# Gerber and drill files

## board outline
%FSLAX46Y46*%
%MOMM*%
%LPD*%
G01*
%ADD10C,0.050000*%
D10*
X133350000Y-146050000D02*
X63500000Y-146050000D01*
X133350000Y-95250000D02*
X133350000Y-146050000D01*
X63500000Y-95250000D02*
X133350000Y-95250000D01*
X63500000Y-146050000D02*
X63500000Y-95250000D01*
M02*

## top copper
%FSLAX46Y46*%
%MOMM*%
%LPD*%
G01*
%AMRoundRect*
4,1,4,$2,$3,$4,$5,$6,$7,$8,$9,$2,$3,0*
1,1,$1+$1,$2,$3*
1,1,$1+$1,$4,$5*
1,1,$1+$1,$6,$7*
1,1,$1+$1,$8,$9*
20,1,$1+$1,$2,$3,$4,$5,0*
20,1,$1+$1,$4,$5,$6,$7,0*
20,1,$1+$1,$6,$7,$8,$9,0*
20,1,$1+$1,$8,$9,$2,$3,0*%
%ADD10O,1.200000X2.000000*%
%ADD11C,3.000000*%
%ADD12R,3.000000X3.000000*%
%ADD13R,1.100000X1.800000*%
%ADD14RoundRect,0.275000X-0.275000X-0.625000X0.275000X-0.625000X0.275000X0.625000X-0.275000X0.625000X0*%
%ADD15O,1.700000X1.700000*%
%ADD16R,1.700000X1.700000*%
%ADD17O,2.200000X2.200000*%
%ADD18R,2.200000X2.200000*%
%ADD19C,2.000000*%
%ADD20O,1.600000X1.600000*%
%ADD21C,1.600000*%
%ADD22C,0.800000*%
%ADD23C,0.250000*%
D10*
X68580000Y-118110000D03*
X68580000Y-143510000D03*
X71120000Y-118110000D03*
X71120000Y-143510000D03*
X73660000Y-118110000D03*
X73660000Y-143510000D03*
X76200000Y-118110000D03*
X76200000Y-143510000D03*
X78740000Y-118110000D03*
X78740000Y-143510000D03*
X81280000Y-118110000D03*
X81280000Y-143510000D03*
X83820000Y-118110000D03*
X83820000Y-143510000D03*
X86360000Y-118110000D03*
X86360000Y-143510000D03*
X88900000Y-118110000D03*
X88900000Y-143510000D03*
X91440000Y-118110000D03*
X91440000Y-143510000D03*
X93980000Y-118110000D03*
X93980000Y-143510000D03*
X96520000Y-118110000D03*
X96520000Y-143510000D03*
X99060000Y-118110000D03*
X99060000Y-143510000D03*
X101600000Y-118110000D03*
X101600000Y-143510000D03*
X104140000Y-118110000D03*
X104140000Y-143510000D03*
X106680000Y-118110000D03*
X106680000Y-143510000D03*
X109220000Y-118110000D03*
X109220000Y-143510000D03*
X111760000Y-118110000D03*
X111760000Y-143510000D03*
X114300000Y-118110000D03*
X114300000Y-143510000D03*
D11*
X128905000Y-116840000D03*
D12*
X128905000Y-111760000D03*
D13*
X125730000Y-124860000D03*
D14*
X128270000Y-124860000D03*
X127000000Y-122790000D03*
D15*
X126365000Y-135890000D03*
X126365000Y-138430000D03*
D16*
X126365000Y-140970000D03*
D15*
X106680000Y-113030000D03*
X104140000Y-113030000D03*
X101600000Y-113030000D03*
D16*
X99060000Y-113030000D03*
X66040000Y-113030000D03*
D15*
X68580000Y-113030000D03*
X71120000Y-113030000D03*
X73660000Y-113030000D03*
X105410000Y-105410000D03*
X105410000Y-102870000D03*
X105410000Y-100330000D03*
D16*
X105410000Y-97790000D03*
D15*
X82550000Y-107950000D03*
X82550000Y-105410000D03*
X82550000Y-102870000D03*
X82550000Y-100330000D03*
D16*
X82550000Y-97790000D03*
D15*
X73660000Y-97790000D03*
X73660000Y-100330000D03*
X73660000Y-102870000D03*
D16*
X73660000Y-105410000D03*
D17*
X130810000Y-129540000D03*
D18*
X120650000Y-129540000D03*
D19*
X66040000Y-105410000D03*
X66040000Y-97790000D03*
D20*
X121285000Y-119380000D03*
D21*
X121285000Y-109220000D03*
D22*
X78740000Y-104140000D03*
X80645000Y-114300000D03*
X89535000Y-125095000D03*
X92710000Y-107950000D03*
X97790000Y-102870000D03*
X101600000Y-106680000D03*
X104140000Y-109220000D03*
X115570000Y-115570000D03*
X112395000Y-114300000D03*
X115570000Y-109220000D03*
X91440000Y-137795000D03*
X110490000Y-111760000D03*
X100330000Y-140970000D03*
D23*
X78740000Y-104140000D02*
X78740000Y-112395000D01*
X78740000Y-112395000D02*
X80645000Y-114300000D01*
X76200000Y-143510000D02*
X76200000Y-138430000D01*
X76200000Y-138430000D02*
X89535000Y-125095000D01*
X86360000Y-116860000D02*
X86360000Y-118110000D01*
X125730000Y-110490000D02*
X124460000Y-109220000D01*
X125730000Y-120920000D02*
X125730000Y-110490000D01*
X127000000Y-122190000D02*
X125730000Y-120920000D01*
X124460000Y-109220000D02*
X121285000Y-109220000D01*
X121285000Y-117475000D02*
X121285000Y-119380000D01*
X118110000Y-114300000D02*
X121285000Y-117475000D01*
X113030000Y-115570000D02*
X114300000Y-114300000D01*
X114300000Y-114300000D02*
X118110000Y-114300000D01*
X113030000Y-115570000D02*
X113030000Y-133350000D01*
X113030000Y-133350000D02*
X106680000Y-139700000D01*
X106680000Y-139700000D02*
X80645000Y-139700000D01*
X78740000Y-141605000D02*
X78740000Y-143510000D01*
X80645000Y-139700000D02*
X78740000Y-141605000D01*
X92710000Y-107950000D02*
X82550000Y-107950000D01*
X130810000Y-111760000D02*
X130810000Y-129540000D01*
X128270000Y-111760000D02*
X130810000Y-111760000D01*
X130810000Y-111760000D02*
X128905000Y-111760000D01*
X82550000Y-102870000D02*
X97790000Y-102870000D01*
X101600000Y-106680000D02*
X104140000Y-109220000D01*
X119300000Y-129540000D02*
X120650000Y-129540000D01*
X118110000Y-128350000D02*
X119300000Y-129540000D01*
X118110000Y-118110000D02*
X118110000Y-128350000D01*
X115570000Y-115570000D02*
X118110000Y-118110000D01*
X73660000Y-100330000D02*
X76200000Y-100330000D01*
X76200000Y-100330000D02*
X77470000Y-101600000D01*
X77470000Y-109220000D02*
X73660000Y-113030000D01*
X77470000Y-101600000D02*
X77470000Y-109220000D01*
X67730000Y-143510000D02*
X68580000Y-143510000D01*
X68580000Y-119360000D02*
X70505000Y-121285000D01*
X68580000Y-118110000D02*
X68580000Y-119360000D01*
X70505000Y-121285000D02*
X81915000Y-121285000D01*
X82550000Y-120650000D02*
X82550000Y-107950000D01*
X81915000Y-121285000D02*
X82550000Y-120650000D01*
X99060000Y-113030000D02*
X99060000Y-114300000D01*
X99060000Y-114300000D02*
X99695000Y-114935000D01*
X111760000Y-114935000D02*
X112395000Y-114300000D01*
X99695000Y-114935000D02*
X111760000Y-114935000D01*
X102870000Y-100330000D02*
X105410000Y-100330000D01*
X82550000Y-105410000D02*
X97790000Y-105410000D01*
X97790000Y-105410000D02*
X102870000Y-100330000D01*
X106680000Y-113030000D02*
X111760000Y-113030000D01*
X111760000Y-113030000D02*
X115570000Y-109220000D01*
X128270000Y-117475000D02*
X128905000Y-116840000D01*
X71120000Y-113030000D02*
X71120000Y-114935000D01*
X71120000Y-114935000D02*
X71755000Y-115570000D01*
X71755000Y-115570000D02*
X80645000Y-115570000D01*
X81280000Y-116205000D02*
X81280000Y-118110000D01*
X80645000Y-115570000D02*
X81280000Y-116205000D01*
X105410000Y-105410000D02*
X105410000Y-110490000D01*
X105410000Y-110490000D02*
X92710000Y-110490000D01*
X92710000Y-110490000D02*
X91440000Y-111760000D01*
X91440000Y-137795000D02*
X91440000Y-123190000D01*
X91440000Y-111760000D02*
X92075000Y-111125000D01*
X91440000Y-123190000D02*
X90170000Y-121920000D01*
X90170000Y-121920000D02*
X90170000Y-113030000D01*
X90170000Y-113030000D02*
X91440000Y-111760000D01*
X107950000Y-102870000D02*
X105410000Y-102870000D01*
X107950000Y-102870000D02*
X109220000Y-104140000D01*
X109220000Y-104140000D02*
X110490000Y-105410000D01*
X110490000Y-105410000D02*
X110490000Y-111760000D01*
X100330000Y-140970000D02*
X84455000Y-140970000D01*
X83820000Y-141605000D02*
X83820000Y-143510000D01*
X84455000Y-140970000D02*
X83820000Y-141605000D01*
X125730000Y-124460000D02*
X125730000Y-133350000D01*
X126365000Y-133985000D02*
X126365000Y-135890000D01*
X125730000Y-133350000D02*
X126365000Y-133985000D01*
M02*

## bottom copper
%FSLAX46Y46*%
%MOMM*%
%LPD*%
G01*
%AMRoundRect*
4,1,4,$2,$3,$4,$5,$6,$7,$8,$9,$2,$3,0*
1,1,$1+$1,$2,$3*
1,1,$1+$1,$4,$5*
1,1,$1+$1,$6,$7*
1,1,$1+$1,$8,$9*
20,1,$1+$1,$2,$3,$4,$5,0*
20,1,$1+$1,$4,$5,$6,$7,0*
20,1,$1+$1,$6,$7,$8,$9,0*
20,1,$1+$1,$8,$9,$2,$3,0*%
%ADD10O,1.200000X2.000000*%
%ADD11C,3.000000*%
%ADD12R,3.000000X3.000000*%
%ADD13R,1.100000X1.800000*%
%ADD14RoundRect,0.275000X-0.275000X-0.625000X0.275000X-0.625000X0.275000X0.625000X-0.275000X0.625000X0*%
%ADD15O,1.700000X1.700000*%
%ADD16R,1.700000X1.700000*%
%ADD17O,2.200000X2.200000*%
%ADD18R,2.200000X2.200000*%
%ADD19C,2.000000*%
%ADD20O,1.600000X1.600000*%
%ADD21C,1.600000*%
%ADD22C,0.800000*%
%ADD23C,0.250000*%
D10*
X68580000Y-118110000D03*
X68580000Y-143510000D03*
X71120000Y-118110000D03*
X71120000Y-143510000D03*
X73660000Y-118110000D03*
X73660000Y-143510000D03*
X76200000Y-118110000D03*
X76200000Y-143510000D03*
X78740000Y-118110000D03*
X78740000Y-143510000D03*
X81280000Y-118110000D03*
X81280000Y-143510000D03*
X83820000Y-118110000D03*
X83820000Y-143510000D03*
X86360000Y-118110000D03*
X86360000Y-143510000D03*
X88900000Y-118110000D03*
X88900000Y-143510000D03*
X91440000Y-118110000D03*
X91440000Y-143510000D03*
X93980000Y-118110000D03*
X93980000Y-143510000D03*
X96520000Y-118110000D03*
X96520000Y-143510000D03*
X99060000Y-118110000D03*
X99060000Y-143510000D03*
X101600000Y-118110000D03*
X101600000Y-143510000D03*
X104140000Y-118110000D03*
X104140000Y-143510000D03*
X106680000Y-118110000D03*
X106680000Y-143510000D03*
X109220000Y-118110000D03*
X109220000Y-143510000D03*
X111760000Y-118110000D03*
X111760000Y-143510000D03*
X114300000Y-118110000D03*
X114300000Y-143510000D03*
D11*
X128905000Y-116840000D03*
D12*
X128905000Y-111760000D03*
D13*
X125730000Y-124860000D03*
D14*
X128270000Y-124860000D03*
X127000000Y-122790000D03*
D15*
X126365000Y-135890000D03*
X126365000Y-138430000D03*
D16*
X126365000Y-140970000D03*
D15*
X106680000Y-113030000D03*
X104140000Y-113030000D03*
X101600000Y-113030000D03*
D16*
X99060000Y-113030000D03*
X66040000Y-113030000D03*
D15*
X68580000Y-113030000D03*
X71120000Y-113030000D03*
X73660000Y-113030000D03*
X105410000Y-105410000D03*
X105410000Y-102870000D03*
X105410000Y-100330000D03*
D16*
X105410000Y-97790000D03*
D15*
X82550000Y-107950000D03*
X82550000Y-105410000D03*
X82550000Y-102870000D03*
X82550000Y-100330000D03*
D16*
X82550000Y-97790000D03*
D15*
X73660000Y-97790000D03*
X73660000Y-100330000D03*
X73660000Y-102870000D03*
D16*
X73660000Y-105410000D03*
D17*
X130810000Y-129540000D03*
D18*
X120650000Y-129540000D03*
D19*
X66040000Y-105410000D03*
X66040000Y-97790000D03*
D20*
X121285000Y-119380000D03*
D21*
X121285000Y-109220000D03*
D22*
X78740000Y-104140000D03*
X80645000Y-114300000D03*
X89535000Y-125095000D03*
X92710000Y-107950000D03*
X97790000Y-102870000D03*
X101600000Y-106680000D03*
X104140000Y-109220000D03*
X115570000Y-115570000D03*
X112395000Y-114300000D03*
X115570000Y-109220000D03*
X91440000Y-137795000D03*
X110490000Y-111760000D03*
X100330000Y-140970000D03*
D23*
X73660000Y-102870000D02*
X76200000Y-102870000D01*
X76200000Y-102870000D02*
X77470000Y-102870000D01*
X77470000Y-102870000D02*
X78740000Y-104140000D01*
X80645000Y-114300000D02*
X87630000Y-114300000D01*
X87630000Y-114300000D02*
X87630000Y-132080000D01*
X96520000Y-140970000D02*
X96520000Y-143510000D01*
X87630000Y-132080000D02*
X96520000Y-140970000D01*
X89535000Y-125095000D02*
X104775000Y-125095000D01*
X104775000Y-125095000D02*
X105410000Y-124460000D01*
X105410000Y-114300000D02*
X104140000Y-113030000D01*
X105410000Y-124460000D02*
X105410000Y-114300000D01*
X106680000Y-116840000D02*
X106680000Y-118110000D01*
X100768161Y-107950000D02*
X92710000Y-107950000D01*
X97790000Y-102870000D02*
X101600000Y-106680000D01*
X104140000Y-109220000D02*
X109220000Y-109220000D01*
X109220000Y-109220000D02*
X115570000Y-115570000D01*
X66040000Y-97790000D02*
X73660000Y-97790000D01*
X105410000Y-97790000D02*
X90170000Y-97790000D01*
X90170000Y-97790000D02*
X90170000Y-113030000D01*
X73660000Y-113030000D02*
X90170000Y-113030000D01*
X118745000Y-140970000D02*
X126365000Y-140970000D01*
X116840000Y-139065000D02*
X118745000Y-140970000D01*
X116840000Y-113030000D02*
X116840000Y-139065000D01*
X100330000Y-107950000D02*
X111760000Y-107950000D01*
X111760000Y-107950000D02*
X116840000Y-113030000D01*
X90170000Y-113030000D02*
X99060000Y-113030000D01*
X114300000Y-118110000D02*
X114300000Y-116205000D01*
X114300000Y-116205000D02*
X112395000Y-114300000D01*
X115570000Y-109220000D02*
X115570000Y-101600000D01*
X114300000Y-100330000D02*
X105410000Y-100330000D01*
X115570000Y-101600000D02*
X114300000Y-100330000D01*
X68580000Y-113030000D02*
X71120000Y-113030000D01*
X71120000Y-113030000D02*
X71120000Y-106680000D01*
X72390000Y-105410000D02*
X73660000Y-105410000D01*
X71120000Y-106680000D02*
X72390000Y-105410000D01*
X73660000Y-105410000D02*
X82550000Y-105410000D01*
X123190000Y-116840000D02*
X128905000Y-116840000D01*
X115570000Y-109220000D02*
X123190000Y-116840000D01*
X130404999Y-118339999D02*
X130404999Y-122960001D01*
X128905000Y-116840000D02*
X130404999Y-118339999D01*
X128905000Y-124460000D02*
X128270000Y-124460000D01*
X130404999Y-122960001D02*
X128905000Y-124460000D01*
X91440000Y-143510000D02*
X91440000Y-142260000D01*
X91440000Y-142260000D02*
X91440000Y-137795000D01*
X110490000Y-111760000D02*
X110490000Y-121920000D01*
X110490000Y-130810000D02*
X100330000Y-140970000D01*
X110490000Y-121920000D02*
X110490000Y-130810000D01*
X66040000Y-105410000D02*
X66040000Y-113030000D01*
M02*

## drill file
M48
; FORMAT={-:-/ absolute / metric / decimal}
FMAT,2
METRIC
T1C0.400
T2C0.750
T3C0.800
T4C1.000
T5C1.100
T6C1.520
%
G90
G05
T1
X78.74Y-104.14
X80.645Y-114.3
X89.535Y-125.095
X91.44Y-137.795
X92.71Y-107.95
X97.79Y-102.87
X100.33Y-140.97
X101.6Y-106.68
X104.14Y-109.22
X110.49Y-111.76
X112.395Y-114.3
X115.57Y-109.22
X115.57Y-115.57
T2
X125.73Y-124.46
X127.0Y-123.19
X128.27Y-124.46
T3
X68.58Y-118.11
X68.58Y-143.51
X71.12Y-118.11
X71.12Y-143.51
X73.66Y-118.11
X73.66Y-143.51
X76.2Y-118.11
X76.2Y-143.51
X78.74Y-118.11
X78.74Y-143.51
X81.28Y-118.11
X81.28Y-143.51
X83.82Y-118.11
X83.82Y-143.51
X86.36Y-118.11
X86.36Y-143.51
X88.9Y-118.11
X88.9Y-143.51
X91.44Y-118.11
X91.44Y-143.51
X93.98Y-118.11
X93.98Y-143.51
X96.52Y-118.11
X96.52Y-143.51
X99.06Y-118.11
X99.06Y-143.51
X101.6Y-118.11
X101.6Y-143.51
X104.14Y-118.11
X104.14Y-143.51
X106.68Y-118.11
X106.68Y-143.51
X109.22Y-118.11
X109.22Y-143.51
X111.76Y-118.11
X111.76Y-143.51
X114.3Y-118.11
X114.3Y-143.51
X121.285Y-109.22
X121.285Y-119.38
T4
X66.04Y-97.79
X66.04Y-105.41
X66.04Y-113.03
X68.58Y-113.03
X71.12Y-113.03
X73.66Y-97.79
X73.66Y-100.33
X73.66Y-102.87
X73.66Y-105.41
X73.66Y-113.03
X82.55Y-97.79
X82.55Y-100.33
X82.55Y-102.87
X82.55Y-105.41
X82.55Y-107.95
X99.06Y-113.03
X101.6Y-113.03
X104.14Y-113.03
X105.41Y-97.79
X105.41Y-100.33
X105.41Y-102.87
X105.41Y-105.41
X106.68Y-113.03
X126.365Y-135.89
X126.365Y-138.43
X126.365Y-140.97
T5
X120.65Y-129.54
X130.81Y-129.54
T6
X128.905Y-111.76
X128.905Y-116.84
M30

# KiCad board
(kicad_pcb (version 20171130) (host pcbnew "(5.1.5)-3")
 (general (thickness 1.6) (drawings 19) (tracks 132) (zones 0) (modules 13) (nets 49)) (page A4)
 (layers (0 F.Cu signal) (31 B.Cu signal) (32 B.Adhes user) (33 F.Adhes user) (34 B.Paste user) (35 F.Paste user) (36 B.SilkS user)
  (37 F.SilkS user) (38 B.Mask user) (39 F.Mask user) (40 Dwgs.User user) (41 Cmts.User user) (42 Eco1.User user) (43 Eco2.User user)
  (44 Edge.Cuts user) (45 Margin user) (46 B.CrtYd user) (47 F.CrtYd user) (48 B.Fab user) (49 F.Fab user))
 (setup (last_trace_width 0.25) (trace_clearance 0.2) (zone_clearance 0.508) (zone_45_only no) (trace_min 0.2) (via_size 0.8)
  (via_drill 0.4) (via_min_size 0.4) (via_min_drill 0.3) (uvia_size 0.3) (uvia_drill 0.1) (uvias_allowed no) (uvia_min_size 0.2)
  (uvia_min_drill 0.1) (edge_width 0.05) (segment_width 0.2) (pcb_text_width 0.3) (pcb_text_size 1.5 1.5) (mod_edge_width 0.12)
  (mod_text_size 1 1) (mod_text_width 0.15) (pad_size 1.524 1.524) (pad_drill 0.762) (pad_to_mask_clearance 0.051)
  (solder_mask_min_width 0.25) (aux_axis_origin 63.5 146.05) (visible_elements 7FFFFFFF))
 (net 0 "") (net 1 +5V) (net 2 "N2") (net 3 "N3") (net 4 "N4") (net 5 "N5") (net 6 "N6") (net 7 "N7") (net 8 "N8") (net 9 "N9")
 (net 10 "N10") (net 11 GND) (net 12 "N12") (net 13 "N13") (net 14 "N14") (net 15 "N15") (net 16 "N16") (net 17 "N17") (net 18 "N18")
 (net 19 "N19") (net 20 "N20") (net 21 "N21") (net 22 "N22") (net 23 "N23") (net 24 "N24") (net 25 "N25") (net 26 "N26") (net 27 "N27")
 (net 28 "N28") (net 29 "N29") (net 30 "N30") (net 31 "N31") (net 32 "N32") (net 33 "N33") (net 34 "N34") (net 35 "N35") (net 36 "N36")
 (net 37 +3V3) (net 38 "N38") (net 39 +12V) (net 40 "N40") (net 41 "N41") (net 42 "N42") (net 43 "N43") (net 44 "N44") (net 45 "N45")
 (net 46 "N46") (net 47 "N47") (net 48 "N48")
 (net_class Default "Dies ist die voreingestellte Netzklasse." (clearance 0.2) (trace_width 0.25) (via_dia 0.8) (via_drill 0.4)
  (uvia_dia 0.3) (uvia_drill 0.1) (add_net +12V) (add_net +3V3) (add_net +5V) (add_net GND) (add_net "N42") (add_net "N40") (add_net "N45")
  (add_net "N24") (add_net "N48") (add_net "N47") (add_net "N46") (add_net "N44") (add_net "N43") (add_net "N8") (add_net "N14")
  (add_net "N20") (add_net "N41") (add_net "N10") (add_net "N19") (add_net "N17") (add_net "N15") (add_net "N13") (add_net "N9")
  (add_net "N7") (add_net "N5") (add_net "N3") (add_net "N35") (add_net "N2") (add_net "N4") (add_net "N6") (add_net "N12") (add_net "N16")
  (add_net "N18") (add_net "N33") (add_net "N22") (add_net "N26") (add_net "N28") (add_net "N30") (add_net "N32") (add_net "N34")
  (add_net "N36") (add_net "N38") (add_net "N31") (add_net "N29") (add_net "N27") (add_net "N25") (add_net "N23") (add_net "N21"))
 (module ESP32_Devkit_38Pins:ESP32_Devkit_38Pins (layer F.Cu) (at 91.44 130.81 180)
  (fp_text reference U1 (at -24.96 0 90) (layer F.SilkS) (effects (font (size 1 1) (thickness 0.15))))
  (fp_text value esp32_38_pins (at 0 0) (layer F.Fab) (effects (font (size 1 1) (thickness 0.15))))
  (pad 19 thru_hole oval (at 22.86 12.7 180) (size 1.2 2) (drill 0.8) (layers *.Cu *.Mask) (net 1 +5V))
  (pad 20 thru_hole oval (at 22.86 -12.7 180) (size 1.2 2) (drill 0.8) (layers *.Cu *.Mask) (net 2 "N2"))
  (pad 18 thru_hole oval (at 20.32 12.7 180) (size 1.2 2) (drill 0.8) (layers *.Cu *.Mask) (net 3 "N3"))
  (pad 21 thru_hole oval (at 20.32 -12.7 180) (size 1.2 2) (drill 0.8) (layers *.Cu *.Mask) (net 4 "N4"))
  (pad 17 thru_hole oval (at 17.78 12.7 180) (size 1.2 2) (drill 0.8) (layers *.Cu *.Mask) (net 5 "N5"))
  (pad 22 thru_hole oval (at 17.78 -12.7 180) (size 1.2 2) (drill 0.8) (layers *.Cu *.Mask) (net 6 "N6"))
  (pad 16 thru_hole oval (at 15.24 12.7 180) (size 1.2 2) (drill 0.8) (layers *.Cu *.Mask) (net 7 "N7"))
  (pad 23 thru_hole oval (at 15.24 -12.7 180) (size 1.2 2) (drill 0.8) (layers *.Cu *.Mask) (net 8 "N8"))
  (pad 15 thru_hole oval (at 12.7 12.7 180) (size 1.2 2) (drill 0.8) (layers *.Cu *.Mask) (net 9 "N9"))
  (pad 24 thru_hole oval (at 12.7 -12.7 180) (size 1.2 2) (drill 0.8) (layers *.Cu *.Mask) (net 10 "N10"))
  (pad 14 thru_hole oval (at 10.16 12.7 180) (size 1.2 2) (drill 0.8) (layers *.Cu *.Mask) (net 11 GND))
  (pad 25 thru_hole oval (at 10.16 -12.7 180) (size 1.2 2) (drill 0.8) (layers *.Cu *.Mask) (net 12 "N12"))
  (pad 13 thru_hole oval (at 7.62 12.7 180) (size 1.2 2) (drill 0.8) (layers *.Cu *.Mask) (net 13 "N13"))
  (pad 26 thru_hole oval (at 7.62 -12.7 180) (size 1.2 2) (drill 0.8) (layers *.Cu *.Mask) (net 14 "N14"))
  (pad 12 thru_hole oval (at 5.08 12.7 180) (size 1.2 2) (drill 0.8) (layers *.Cu *.Mask) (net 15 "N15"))
  (pad 27 thru_hole oval (at 5.08 -12.7 180) (size 1.2 2) (drill 0.8) (layers *.Cu *.Mask) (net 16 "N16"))
  (pad 11 thru_hole oval (at 2.54 12.7 180) (size 1.2 2) (drill 0.8) (layers *.Cu *.Mask) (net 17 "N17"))
  (pad 28 thru_hole oval (at 2.54 -12.7 180) (size 1.2 2) (drill 0.8) (layers *.Cu *.Mask) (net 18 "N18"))
  (pad 10 thru_hole oval (at 0 12.7 180) (size 1.2 2) (drill 0.8) (layers *.Cu *.Mask) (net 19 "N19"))
  (pad 29 thru_hole oval (at 0 -12.7 180) (size 1.2 2) (drill 0.8) (layers *.Cu *.Mask) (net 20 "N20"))
  (pad 9 thru_hole oval (at -2.54 12.7 180) (size 1.2 2) (drill 0.8) (layers *.Cu *.Mask) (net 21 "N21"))
  (pad 30 thru_hole oval (at -2.54 -12.7 180) (size 1.2 2) (drill 0.8) (layers *.Cu *.Mask) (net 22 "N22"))
  (pad 8 thru_hole oval (at -5.08 12.7 180) (size 1.2 2) (drill 0.8) (layers *.Cu *.Mask) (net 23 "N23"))
  (pad 31 thru_hole oval (at -5.08 -12.7 180) (size 1.2 2) (drill 0.8) (layers *.Cu *.Mask) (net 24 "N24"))
  (pad 7 thru_hole oval (at -7.62 12.7 180) (size 1.2 2) (drill 0.8) (layers *.Cu *.Mask) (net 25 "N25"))
  (pad 32 thru_hole oval (at -7.62 -12.7 180) (size 1.2 2) (drill 0.8) (layers *.Cu *.Mask) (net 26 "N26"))
  (pad 6 thru_hole oval (at -10.16 12.7 180) (size 1.2 2) (drill 0.8) (layers *.Cu *.Mask) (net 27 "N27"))
  (pad 33 thru_hole oval (at -10.16 -12.7 180) (size 1.2 2) (drill 0.8) (layers *.Cu *.Mask) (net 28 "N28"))
  (pad 5 thru_hole oval (at -12.7 12.7 180) (size 1.2 2) (drill 0.8) (layers *.Cu *.Mask) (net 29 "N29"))
  (pad 34 thru_hole oval (at -12.7 -12.7 180) (size 1.2 2) (drill 0.8) (layers *.Cu *.Mask) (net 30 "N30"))
  (pad 4 thru_hole oval (at -15.24 12.7 180) (size 1.2 2) (drill 0.8) (layers *.Cu *.Mask) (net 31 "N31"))
  (pad 35 thru_hole oval (at -15.24 -12.7 180) (size 1.2 2) (drill 0.8) (layers *.Cu *.Mask) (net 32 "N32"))
  (pad 3 thru_hole oval (at -17.78 12.7 180) (size 1.2 2) (drill 0.8) (layers *.Cu *.Mask) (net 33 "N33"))
  (pad 36 thru_hole oval (at -17.78 -12.7 180) (size 1.2 2) (drill 0.8) (layers *.Cu *.Mask) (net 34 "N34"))
  (pad 2 thru_hole oval (at -20.32 12.7 180) (size 1.2 2) (drill 0.8) (layers *.Cu *.Mask) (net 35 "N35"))
  (pad 37 thru_hole oval (at -20.32 -12.7 180) (size 1.2 2) (drill 0.8) (layers *.Cu *.Mask) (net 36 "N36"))
  (pad 1 thru_hole oval (at -22.86 12.7 180) (size 1.2 2) (drill 0.8) (layers *.Cu *.Mask) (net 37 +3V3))
  (pad 38 thru_hole oval (at -22.86 -12.7 180) (size 1.2 2) (drill 0.8) (layers *.Cu *.Mask) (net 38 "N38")))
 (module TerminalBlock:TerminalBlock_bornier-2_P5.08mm (layer F.Cu) (at 128.905 111.76 270)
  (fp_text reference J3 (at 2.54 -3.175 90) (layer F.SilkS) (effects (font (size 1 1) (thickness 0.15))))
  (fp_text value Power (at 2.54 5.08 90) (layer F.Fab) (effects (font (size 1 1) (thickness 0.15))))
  (pad 2 thru_hole circle (at 5.08 0 270) (size 3 3) (drill 1.52) (layers *.Cu *.Mask) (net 11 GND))
  (pad 1 thru_hole rect (at 0 0 270) (size 3 3) (drill 1.52) (layers *.Cu *.Mask) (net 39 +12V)))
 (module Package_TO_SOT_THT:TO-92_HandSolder (layer F.Cu) (at 125.73 124.46)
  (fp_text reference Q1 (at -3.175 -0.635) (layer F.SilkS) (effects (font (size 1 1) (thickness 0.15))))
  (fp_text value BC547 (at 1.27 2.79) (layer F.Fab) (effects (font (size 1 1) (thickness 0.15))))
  (pad 1 thru_hole rect (at 0 0) (size 1.1 1.8) (drill 0.75 (offset 0 0.4)) (layers *.Cu *.Mask) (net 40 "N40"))
  (pad 3 thru_hole roundrect (at 2.54 0) (size 1.1 1.8) (drill 0.75 (offset 0 0.4)) (layers *.Cu *.Mask) (roundrect_rratio 0.25)
   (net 11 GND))
  (pad 2 thru_hole roundrect (at 1.27 -1.27) (size 1.1 1.8) (drill 0.75 (offset 0 -0.4)) (layers *.Cu *.Mask) (roundrect_rratio 0.25)
   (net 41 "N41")))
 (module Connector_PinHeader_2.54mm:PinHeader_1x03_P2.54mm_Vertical (layer F.Cu) (at 126.365 140.97 180)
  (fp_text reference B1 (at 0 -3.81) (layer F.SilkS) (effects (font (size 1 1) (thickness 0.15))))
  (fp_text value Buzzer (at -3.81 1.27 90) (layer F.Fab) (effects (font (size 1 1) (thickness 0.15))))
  (pad 3 thru_hole oval (at 0 5.08 180) (size 1.7 1.7) (drill 1) (layers *.Cu *.Mask) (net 40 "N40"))
  (pad 2 thru_hole oval (at 0 2.54 180) (size 1.7 1.7) (drill 1) (layers *.Cu *.Mask) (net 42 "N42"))
  (pad 1 thru_hole rect (at 0 0 180) (size 1.7 1.7) (drill 1) (layers *.Cu *.Mask) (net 1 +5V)))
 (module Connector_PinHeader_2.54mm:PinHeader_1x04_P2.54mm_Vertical (layer F.Cu) (at 99.06 113.03 90)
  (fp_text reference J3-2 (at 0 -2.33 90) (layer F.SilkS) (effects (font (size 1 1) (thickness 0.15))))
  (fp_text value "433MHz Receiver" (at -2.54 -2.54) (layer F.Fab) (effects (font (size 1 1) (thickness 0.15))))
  (pad 4 thru_hole oval (at 0 7.62 90) (size 1.7 1.7) (drill 1) (layers *.Cu *.Mask) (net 11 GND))
  (pad 3 thru_hole oval (at 0 5.08 90) (size 1.7 1.7) (drill 1) (layers *.Cu *.Mask) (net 8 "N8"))
  (pad 2 thru_hole oval (at 0 2.54 90) (size 1.7 1.7) (drill 1) (layers *.Cu *.Mask) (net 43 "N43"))
  (pad 1 thru_hole rect (at 0 0 90) (size 1.7 1.7) (drill 1) (layers *.Cu *.Mask) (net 37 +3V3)))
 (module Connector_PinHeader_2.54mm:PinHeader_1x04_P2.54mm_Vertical (layer F.Cu) (at 66.04 113.03 90)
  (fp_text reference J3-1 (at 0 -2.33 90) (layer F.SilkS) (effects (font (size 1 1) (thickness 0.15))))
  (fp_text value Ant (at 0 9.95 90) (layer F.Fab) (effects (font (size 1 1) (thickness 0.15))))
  (pad 1 thru_hole rect (at 0 0 90) (size 1.7 1.7) (drill 1) (layers *.Cu *.Mask) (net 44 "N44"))
  (pad 2 thru_hole oval (at 0 2.54 90) (size 1.7 1.7) (drill 1) (layers *.Cu *.Mask) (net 11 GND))
  (pad 3 thru_hole oval (at 0 5.08 90) (size 1.7 1.7) (drill 1) (layers *.Cu *.Mask) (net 11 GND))
  (pad 4 thru_hole oval (at 0 7.62 90) (size 1.7 1.7) (drill 1) (layers *.Cu *.Mask) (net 37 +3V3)))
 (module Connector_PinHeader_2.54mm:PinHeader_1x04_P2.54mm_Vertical (layer F.Cu) (at 105.41 97.79)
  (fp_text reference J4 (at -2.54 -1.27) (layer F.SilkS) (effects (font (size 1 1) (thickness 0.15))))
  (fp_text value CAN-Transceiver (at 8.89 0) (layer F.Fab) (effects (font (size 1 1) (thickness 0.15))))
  (pad 4 thru_hole oval (at 0 7.62) (size 1.7 1.7) (drill 1) (layers *.Cu *.Mask) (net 20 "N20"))
  (pad 3 thru_hole oval (at 0 5.08) (size 1.7 1.7) (drill 1) (layers *.Cu *.Mask) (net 14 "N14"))
  (pad 2 thru_hole oval (at 0 2.54) (size 1.7 1.7) (drill 1) (layers *.Cu *.Mask) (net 11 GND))
  (pad 1 thru_hole rect (at 0 0) (size 1.7 1.7) (drill 1) (layers *.Cu *.Mask) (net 37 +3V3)))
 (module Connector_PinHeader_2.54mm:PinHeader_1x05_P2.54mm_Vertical (layer F.Cu) (at 82.55 97.79)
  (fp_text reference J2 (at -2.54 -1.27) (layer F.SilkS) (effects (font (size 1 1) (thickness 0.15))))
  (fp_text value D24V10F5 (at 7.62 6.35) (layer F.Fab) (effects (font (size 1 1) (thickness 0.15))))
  (pad 5 thru_hole oval (at 0 10.16) (size 1.7 1.7) (drill 1) (layers *.Cu *.Mask) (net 1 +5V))
  (pad 4 thru_hole oval (at 0 7.62) (size 1.7 1.7) (drill 1) (layers *.Cu *.Mask) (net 11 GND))
  (pad 3 thru_hole oval (at 0 5.08) (size 1.7 1.7) (drill 1) (layers *.Cu *.Mask) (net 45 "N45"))
  (pad 2 thru_hole oval (at 0 2.54) (size 1.7 1.7) (drill 1) (layers *.Cu *.Mask) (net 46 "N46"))
  (pad 1 thru_hole rect (at 0 0) (size 1.7 1.7) (drill 1) (layers *.Cu *.Mask) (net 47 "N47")))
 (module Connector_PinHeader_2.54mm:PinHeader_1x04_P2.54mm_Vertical (layer F.Cu) (at 73.66 105.41 180)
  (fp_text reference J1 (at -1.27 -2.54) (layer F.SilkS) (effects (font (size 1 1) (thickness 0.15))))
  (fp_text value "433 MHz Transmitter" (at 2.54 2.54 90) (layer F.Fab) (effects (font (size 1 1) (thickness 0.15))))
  (pad 4 thru_hole oval (at 0 7.62 180) (size 1.7 1.7) (drill 1) (layers *.Cu *.Mask) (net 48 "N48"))
  (pad 3 thru_hole oval (at 0 5.08 180) (size 1.7 1.7) (drill 1) (layers *.Cu *.Mask) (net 37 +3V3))
  (pad 2 thru_hole oval (at 0 2.54 180) (size 1.7 1.7) (drill 1) (layers *.Cu *.Mask) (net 24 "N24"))
  (pad 1 thru_hole rect (at 0 0 180) (size 1.7 1.7) (drill 1) (layers *.Cu *.Mask) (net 11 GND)))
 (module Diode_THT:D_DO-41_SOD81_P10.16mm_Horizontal (layer F.Cu) (at 120.65 129.54)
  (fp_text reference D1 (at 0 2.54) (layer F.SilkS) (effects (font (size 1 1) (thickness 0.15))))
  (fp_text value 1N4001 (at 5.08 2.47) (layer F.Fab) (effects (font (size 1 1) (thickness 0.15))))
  (pad 2 thru_hole oval (at 10.16 0) (size 2.2 2.2) (drill 1.1) (layers *.Cu *.Mask) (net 39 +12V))
  (pad 1 thru_hole rect (at 0 0) (size 2.2 2.2) (drill 1.1) (layers *.Cu *.Mask) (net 45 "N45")))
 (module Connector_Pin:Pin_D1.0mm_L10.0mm (layer F.Cu) (at 66.04 105.41)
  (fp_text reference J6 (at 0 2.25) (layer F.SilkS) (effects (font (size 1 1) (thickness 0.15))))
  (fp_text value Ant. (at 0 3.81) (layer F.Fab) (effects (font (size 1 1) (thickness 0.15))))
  (pad 1 thru_hole circle (at 0 0) (size 2 2) (drill 1) (layers *.Cu *.Mask) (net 44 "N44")))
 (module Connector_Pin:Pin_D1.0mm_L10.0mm (layer F.Cu) (at 66.04 97.79)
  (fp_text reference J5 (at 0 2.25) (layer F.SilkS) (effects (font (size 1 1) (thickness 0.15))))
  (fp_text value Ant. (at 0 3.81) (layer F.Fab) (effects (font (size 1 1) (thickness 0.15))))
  (pad 1 thru_hole circle (at 0 0) (size 2 2) (drill 1) (layers *.Cu *.Mask) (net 48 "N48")))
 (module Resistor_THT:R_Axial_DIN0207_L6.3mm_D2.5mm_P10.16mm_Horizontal (layer F.Cu) (at 121.285 109.22 270)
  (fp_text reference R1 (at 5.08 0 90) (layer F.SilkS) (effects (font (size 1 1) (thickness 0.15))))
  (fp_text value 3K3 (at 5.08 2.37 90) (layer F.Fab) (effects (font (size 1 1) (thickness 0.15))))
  (pad 2 thru_hole oval (at 10.16 0 270) (size 1.6 1.6) (drill 0.8) (layers *.Cu *.Mask) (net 10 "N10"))
  (pad 1 thru_hole circle (at 0 0 270) (size 1.6 1.6) (drill 0.8) (layers *.Cu *.Mask) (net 41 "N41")))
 (gr_line (start 133.35 146.05) (end 63.5 146.05) (layer Edge.Cuts) (width 0.05))
 (gr_line (start 133.35 95.25) (end 133.35 146.05) (layer Edge.Cuts) (width 0.05))
 (gr_line (start 63.5 95.25) (end 133.35 95.25) (layer Edge.Cuts) (width 0.05))
 (gr_line (start 63.5 146.05) (end 63.5 95.25) (layer Edge.Cuts) (width 0.05))
 (segment (start 73.66 102.87) (end 76.2 102.87) (width 0.25) (layer B.Cu) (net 24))
 (segment (start 76.2 102.87) (end 77.47 102.87) (width 0.25) (layer B.Cu) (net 24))
 (via (at 78.74 104.14) (size 0.8) (drill 0.4) (layers F.Cu B.Cu) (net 24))
 (segment (start 77.47 102.87) (end 78.74 104.14) (width 0.25) (layer B.Cu) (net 24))
 (segment (start 78.74 104.14) (end 78.74 112.395) (width 0.25) (layer F.Cu) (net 24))
 (via (at 80.645 114.3) (size 0.8) (drill 0.4) (layers F.Cu B.Cu) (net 24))
 (segment (start 78.74 112.395) (end 80.645 114.3) (width 0.25) (layer F.Cu) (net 24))
 (segment (start 80.645 114.3) (end 87.63 114.3) (width 0.25) (layer B.Cu) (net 24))
 (segment (start 87.63 114.3) (end 87.63 132.08) (width 0.25) (layer B.Cu) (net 24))
 (segment (start 96.52 140.97) (end 96.52 143.51) (width 0.25) (layer B.Cu) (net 24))
 (segment (start 87.63 132.08) (end 96.52 140.97) (width 0.25) (layer B.Cu) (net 24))
 (segment (start 76.2 143.51) (end 76.2 138.43) (width 0.25) (layer F.Cu) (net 8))
 (via (at 89.535 125.095) (size 0.8) (drill 0.4) (layers F.Cu B.Cu) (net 8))
 (segment (start 76.2 138.43) (end 89.535 125.095) (width 0.25) (layer F.Cu) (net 8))
 (segment (start 89.535 125.095) (end 104.775 125.095) (width 0.25) (layer B.Cu) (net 8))
 (segment (start 104.775 125.095) (end 105.41 124.46) (width 0.25) (layer B.Cu) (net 8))
 (segment (start 105.41 114.3) (end 104.14 113.03) (width 0.25) (layer B.Cu) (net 8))
 (segment (start 105.41 124.46) (end 105.41 114.3) (width 0.25) (layer B.Cu) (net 8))
 (segment (start 86.36 116.86) (end 86.36 118.11) (width 0.25) (layer F.Cu) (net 15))
 (segment (start 106.68 116.84) (end 106.68 118.11) (width 0.25) (layer B.Cu) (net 31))
 (segment (start 125.73 110.49) (end 124.46 109.22) (width 0.25) (layer F.Cu) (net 41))
 (segment (start 125.73 120.92) (end 125.73 110.49) (width 0.25) (layer F.Cu) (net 41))
 (segment (start 127 122.19) (end 125.73 120.92) (width 0.25) (layer F.Cu) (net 41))
 (segment (start 124.46 109.22) (end 121.285 109.22) (width 0.25) (layer F.Cu) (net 41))
 (segment (start 121.285 117.475) (end 121.285 119.38) (width 0.25) (layer F.Cu) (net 10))
 (segment (start 118.11 114.3) (end 121.285 117.475) (width 0.25) (layer F.Cu) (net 10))
 (segment (start 113.03 115.57) (end 114.3 114.3) (width 0.25) (layer F.Cu) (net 10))
 (segment (start 114.3 114.3) (end 118.11 114.3) (width 0.25) (layer F.Cu) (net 10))
 (segment (start 113.03 115.57) (end 113.03 133.35) (width 0.25) (layer F.Cu) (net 10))
 (segment (start 113.03 133.35) (end 106.68 139.7) (width 0.25) (layer F.Cu) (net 10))
 (segment (start 106.68 139.7) (end 80.645 139.7) (width 0.25) (layer F.Cu) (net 10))
 (segment (start 78.74 141.605) (end 78.74 143.51) (width 0.25) (layer F.Cu) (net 10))
 (segment (start 80.645 139.7) (end 78.74 141.605) (width 0.25) (layer F.Cu) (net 10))
 (segment (start 100.768161 107.95) (end 92.71 107.95) (width 0.25) (layer B.Cu) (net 1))
 (via (at 92.71 107.95) (size 0.8) (drill 0.4) (layers F.Cu B.Cu) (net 1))
 (segment (start 92.71 107.95) (end 82.55 107.95) (width 0.25) (layer F.Cu) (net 1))
 (segment (start 130.81 111.76) (end 130.81 129.54) (width 0.25) (layer F.Cu) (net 39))
 (segment (start 128.27 111.76) (end 130.81 111.76) (width 0.25) (layer F.Cu) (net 39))
 (segment (start 130.81 111.76) (end 128.905 111.76) (width 0.25) (layer F.Cu) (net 39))
 (segment (start 82.55 102.87) (end 97.79 102.87) (width 0.25) (layer F.Cu) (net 45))
 (via (at 97.79 102.87) (size 0.8) (drill 0.4) (layers F.Cu B.Cu) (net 45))
 (segment (start 97.79 102.87) (end 101.6 106.68) (width 0.25) (layer B.Cu) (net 45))
 (via (at 101.6 106.68) (size 0.8) (drill 0.4) (layers F.Cu B.Cu) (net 45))
 (segment (start 101.6 106.68) (end 104.14 109.22) (width 0.25) (layer F.Cu) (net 45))
 (via (at 104.14 109.22) (size 0.8) (drill 0.4) (layers F.Cu B.Cu) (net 45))
 (segment (start 104.14 109.22) (end 109.22 109.22) (width 0.25) (layer B.Cu) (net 45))
 (segment (start 109.22 109.22) (end 115.57 115.57) (width 0.25) (layer B.Cu) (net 45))
 (via (at 115.57 115.57) (size 0.8) (drill 0.4) (layers F.Cu B.Cu) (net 45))
 (segment (start 119.3 129.54) (end 120.65 129.54) (width 0.25) (layer F.Cu) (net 45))
 (segment (start 118.11 128.35) (end 119.3 129.54) (width 0.25) (layer F.Cu) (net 45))
 (segment (start 118.11 118.11) (end 118.11 128.35) (width 0.25) (layer F.Cu) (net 45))
 (segment (start 115.57 115.57) (end 118.11 118.11) (width 0.25) (layer F.Cu) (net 45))
 (segment (start 66.04 97.79) (end 73.66 97.79) (width 0.25) (layer B.Cu) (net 48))
 (segment (start 105.41 97.79) (end 90.17 97.79) (width 0.25) (layer B.Cu) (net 37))
 (segment (start 90.17 97.79) (end 90.17 113.03) (width 0.25) (layer B.Cu) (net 37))
 (segment (start 73.66 113.03) (end 90.17 113.03) (width 0.25) (layer B.Cu) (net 37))
 (segment (start 73.66 100.33) (end 76.2 100.33) (width 0.25) (layer F.Cu) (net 37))
 (segment (start 76.2 100.33) (end 77.47 101.6) (width 0.25) (layer F.Cu) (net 37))
 (segment (start 77.47 109.22) (end 73.66 113.03) (width 0.25) (layer F.Cu) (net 37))
 (segment (start 77.47 101.6) (end 77.47 109.22) (width 0.25) (layer F.Cu) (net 37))
 (segment (start 67.73 143.51) (end 68.58 143.51) (width 0.25) (layer F.Cu) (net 2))
 (segment (start 68.58 119.36) (end 70.505 121.285) (width 0.25) (layer F.Cu) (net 1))
 (segment (start 68.58 118.11) (end 68.58 119.36) (width 0.25) (layer F.Cu) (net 1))
 (segment (start 70.505 121.285) (end 81.915 121.285) (width 0.25) (layer F.Cu) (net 1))
 (segment (start 82.55 120.65) (end 82.55 107.95) (width 0.25) (layer F.Cu) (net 1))
 (segment (start 81.915 121.285) (end 82.55 120.65) (width 0.25) (layer F.Cu) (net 1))
 (segment (start 118.745 140.97) (end 126.365 140.97) (width 0.25) (layer B.Cu) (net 1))
 (segment (start 116.84 139.065) (end 118.745 140.97) (width 0.25) (layer B.Cu) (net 1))
 (segment (start 116.84 113.03) (end 116.84 139.065) (width 0.25) (layer B.Cu) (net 1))
 (segment (start 100.33 107.95) (end 111.76 107.95) (width 0.25) (layer B.Cu) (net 1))
 (segment (start 111.76 107.95) (end 116.84 113.03) (width 0.25) (layer B.Cu) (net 1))
 (segment (start 90.17 113.03) (end 99.06 113.03) (width 0.25) (layer B.Cu) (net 37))
 (segment (start 114.3 118.11) (end 114.3 116.205) (width 0.25) (layer B.Cu) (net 37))
 (segment (start 114.3 116.205) (end 112.395 114.3) (width 0.25) (layer B.Cu) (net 37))
 (via (at 112.395 114.3) (size 0.8) (drill 0.4) (layers F.Cu B.Cu) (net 37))
 (segment (start 99.06 113.03) (end 99.06 114.3) (width 0.25) (layer F.Cu) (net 37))
 (segment (start 99.06 114.3) (end 99.695 114.935) (width 0.25) (layer F.Cu) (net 37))
 (segment (start 111.76 114.935) (end 112.395 114.3) (width 0.25) (layer F.Cu) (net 37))
 (segment (start 99.695 114.935) (end 111.76 114.935) (width 0.25) (layer F.Cu) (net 37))
 (segment (start 115.57 109.22) (end 115.57 101.6) (width 0.25) (layer B.Cu) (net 11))
 (segment (start 114.3 100.33) (end 105.41 100.33) (width 0.25) (layer B.Cu) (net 11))
 (segment (start 115.57 101.6) (end 114.3 100.33) (width 0.25) (layer B.Cu) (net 11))
 (segment (start 68.58 113.03) (end 71.12 113.03) (width 0.25) (layer B.Cu) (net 11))
 (segment (start 71.12 113.03) (end 71.12 106.68) (width 0.25) (layer B.Cu) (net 11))
 (segment (start 72.39 105.41) (end 73.66 105.41) (width 0.25) (layer B.Cu) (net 11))
 (segment (start 71.12 106.68) (end 72.39 105.41) (width 0.25) (layer B.Cu) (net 11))
 (segment (start 73.66 105.41) (end 82.55 105.41) (width 0.25) (layer B.Cu) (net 11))
 (segment (start 102.87 100.33) (end 105.41 100.33) (width 0.25) (layer F.Cu) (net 11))
 (segment (start 82.55 105.41) (end 97.79 105.41) (width 0.25) (layer F.Cu) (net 11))
 (segment (start 97.79 105.41) (end 102.87 100.33) (width 0.25) (layer F.Cu) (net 11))
 (segment (start 106.68 113.03) (end 111.76 113.03) (width 0.25) (layer F.Cu) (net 11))
 (segment (start 111.76 113.03) (end 115.57 109.22) (width 0.25) (layer F.Cu) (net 11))
 (via (at 115.57 109.22) (size 0.8) (drill 0.4) (layers F.Cu B.Cu) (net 11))
 (segment (start 123.19 116.84) (end 128.905 116.84) (width 0.25) (layer B.Cu) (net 11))
 (segment (start 115.57 109.22) (end 123.19 116.84) (width 0.25) (layer B.Cu) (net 11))
 (segment (start 128.27 117.475) (end 128.905 116.84) (width 0.25) (layer F.Cu) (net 11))
 (segment (start 130.404999 118.339999) (end 130.404999 122.960001) (width 0.25) (layer B.Cu) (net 11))
 (segment (start 128.905 116.84) (end 130.404999 118.339999) (width 0.25) (layer B.Cu) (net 11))
 (segment (start 128.905 124.46) (end 128.27 124.46) (width 0.25) (layer B.Cu) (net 11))
 (segment (start 130.404999 122.960001) (end 128.905 124.46) (width 0.25) (layer B.Cu) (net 11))
 (segment (start 71.12 113.03) (end 71.12 114.935) (width 0.25) (layer F.Cu) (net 11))
 (segment (start 71.12 114.935) (end 71.755 115.57) (width 0.25) (layer F.Cu) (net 11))
 (segment (start 71.755 115.57) (end 80.645 115.57) (width 0.25) (layer F.Cu) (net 11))
 (segment (start 81.28 116.205) (end 81.28 118.11) (width 0.25) (layer F.Cu) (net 11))
 (segment (start 80.645 115.57) (end 81.28 116.205) (width 0.25) (layer F.Cu) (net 11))
 (segment (start 105.41 105.41) (end 105.41 110.49) (width 0.25) (layer F.Cu) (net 20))
 (segment (start 105.41 110.49) (end 92.71 110.49) (width 0.25) (layer F.Cu) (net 20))
 (segment (start 92.71 110.49) (end 91.44 111.76) (width 0.25) (layer F.Cu) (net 20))
 (segment (start 91.44 143.51) (end 91.44 142.26) (width 0.25) (layer B.Cu) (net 20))
 (via (at 91.44 137.795) (size 0.8) (drill 0.4) (layers F.Cu B.Cu) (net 20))
 (segment (start 91.44 142.26) (end 91.44 137.795) (width 0.25) (layer B.Cu) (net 20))
 (segment (start 91.44 137.795) (end 91.44 123.19) (width 0.25) (layer F.Cu) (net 20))
 (segment (start 91.44 111.76) (end 92.075 111.125) (width 0.25) (layer F.Cu) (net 20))
 (segment (start 91.44 123.19) (end 90.17 121.92) (width 0.25) (layer F.Cu) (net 20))
 (segment (start 90.17 121.92) (end 90.17 113.03) (width 0.25) (layer F.Cu) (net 20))
 (segment (start 90.17 113.03) (end 91.44 111.76) (width 0.25) (layer F.Cu) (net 20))
 (segment (start 107.95 102.87) (end 105.41 102.87) (width 0.25) (layer F.Cu) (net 14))
 (segment (start 107.95 102.87) (end 109.22 104.14) (width 0.25) (layer F.Cu) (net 14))
 (segment (start 109.22 104.14) (end 110.49 105.41) (width 0.25) (layer F.Cu) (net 14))
 (via (at 110.49 111.76) (size 0.8) (drill 0.4) (layers F.Cu B.Cu) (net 14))
 (segment (start 110.49 105.41) (end 110.49 111.76) (width 0.25) (layer F.Cu) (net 14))
 (segment (start 110.49 111.76) (end 110.49 121.92) (width 0.25) (layer B.Cu) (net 14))
 (segment (start 110.49 130.81) (end 100.33 140.97) (width 0.25) (layer B.Cu) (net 14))
 (segment (start 110.49 121.92) (end 110.49 130.81) (width 0.25) (layer B.Cu) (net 14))
 (via (at 100.33 140.97) (size 0.8) (drill 0.4) (layers F.Cu B.Cu) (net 14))
 (segment (start 100.33 140.97) (end 84.455 140.97) (width 0.25) (layer F.Cu) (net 14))
 (segment (start 83.82 141.605) (end 83.82 143.51) (width 0.25) (layer F.Cu) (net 14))
 (segment (start 84.455 140.97) (end 83.82 141.605) (width 0.25) (layer F.Cu) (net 14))
 (segment (start 66.04 105.41) (end 66.04 113.03) (width 0.25) (layer B.Cu) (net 44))
 (segment (start 125.73 124.46) (end 125.73 133.35) (width 0.25) (layer F.Cu) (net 40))
 (segment (start 126.365 133.985) (end 126.365 135.89) (width 0.25) (layer F.Cu) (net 40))
 (segment (start 125.73 133.35) (end 126.365 133.985) (width 0.25) (layer F.Cu) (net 40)))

